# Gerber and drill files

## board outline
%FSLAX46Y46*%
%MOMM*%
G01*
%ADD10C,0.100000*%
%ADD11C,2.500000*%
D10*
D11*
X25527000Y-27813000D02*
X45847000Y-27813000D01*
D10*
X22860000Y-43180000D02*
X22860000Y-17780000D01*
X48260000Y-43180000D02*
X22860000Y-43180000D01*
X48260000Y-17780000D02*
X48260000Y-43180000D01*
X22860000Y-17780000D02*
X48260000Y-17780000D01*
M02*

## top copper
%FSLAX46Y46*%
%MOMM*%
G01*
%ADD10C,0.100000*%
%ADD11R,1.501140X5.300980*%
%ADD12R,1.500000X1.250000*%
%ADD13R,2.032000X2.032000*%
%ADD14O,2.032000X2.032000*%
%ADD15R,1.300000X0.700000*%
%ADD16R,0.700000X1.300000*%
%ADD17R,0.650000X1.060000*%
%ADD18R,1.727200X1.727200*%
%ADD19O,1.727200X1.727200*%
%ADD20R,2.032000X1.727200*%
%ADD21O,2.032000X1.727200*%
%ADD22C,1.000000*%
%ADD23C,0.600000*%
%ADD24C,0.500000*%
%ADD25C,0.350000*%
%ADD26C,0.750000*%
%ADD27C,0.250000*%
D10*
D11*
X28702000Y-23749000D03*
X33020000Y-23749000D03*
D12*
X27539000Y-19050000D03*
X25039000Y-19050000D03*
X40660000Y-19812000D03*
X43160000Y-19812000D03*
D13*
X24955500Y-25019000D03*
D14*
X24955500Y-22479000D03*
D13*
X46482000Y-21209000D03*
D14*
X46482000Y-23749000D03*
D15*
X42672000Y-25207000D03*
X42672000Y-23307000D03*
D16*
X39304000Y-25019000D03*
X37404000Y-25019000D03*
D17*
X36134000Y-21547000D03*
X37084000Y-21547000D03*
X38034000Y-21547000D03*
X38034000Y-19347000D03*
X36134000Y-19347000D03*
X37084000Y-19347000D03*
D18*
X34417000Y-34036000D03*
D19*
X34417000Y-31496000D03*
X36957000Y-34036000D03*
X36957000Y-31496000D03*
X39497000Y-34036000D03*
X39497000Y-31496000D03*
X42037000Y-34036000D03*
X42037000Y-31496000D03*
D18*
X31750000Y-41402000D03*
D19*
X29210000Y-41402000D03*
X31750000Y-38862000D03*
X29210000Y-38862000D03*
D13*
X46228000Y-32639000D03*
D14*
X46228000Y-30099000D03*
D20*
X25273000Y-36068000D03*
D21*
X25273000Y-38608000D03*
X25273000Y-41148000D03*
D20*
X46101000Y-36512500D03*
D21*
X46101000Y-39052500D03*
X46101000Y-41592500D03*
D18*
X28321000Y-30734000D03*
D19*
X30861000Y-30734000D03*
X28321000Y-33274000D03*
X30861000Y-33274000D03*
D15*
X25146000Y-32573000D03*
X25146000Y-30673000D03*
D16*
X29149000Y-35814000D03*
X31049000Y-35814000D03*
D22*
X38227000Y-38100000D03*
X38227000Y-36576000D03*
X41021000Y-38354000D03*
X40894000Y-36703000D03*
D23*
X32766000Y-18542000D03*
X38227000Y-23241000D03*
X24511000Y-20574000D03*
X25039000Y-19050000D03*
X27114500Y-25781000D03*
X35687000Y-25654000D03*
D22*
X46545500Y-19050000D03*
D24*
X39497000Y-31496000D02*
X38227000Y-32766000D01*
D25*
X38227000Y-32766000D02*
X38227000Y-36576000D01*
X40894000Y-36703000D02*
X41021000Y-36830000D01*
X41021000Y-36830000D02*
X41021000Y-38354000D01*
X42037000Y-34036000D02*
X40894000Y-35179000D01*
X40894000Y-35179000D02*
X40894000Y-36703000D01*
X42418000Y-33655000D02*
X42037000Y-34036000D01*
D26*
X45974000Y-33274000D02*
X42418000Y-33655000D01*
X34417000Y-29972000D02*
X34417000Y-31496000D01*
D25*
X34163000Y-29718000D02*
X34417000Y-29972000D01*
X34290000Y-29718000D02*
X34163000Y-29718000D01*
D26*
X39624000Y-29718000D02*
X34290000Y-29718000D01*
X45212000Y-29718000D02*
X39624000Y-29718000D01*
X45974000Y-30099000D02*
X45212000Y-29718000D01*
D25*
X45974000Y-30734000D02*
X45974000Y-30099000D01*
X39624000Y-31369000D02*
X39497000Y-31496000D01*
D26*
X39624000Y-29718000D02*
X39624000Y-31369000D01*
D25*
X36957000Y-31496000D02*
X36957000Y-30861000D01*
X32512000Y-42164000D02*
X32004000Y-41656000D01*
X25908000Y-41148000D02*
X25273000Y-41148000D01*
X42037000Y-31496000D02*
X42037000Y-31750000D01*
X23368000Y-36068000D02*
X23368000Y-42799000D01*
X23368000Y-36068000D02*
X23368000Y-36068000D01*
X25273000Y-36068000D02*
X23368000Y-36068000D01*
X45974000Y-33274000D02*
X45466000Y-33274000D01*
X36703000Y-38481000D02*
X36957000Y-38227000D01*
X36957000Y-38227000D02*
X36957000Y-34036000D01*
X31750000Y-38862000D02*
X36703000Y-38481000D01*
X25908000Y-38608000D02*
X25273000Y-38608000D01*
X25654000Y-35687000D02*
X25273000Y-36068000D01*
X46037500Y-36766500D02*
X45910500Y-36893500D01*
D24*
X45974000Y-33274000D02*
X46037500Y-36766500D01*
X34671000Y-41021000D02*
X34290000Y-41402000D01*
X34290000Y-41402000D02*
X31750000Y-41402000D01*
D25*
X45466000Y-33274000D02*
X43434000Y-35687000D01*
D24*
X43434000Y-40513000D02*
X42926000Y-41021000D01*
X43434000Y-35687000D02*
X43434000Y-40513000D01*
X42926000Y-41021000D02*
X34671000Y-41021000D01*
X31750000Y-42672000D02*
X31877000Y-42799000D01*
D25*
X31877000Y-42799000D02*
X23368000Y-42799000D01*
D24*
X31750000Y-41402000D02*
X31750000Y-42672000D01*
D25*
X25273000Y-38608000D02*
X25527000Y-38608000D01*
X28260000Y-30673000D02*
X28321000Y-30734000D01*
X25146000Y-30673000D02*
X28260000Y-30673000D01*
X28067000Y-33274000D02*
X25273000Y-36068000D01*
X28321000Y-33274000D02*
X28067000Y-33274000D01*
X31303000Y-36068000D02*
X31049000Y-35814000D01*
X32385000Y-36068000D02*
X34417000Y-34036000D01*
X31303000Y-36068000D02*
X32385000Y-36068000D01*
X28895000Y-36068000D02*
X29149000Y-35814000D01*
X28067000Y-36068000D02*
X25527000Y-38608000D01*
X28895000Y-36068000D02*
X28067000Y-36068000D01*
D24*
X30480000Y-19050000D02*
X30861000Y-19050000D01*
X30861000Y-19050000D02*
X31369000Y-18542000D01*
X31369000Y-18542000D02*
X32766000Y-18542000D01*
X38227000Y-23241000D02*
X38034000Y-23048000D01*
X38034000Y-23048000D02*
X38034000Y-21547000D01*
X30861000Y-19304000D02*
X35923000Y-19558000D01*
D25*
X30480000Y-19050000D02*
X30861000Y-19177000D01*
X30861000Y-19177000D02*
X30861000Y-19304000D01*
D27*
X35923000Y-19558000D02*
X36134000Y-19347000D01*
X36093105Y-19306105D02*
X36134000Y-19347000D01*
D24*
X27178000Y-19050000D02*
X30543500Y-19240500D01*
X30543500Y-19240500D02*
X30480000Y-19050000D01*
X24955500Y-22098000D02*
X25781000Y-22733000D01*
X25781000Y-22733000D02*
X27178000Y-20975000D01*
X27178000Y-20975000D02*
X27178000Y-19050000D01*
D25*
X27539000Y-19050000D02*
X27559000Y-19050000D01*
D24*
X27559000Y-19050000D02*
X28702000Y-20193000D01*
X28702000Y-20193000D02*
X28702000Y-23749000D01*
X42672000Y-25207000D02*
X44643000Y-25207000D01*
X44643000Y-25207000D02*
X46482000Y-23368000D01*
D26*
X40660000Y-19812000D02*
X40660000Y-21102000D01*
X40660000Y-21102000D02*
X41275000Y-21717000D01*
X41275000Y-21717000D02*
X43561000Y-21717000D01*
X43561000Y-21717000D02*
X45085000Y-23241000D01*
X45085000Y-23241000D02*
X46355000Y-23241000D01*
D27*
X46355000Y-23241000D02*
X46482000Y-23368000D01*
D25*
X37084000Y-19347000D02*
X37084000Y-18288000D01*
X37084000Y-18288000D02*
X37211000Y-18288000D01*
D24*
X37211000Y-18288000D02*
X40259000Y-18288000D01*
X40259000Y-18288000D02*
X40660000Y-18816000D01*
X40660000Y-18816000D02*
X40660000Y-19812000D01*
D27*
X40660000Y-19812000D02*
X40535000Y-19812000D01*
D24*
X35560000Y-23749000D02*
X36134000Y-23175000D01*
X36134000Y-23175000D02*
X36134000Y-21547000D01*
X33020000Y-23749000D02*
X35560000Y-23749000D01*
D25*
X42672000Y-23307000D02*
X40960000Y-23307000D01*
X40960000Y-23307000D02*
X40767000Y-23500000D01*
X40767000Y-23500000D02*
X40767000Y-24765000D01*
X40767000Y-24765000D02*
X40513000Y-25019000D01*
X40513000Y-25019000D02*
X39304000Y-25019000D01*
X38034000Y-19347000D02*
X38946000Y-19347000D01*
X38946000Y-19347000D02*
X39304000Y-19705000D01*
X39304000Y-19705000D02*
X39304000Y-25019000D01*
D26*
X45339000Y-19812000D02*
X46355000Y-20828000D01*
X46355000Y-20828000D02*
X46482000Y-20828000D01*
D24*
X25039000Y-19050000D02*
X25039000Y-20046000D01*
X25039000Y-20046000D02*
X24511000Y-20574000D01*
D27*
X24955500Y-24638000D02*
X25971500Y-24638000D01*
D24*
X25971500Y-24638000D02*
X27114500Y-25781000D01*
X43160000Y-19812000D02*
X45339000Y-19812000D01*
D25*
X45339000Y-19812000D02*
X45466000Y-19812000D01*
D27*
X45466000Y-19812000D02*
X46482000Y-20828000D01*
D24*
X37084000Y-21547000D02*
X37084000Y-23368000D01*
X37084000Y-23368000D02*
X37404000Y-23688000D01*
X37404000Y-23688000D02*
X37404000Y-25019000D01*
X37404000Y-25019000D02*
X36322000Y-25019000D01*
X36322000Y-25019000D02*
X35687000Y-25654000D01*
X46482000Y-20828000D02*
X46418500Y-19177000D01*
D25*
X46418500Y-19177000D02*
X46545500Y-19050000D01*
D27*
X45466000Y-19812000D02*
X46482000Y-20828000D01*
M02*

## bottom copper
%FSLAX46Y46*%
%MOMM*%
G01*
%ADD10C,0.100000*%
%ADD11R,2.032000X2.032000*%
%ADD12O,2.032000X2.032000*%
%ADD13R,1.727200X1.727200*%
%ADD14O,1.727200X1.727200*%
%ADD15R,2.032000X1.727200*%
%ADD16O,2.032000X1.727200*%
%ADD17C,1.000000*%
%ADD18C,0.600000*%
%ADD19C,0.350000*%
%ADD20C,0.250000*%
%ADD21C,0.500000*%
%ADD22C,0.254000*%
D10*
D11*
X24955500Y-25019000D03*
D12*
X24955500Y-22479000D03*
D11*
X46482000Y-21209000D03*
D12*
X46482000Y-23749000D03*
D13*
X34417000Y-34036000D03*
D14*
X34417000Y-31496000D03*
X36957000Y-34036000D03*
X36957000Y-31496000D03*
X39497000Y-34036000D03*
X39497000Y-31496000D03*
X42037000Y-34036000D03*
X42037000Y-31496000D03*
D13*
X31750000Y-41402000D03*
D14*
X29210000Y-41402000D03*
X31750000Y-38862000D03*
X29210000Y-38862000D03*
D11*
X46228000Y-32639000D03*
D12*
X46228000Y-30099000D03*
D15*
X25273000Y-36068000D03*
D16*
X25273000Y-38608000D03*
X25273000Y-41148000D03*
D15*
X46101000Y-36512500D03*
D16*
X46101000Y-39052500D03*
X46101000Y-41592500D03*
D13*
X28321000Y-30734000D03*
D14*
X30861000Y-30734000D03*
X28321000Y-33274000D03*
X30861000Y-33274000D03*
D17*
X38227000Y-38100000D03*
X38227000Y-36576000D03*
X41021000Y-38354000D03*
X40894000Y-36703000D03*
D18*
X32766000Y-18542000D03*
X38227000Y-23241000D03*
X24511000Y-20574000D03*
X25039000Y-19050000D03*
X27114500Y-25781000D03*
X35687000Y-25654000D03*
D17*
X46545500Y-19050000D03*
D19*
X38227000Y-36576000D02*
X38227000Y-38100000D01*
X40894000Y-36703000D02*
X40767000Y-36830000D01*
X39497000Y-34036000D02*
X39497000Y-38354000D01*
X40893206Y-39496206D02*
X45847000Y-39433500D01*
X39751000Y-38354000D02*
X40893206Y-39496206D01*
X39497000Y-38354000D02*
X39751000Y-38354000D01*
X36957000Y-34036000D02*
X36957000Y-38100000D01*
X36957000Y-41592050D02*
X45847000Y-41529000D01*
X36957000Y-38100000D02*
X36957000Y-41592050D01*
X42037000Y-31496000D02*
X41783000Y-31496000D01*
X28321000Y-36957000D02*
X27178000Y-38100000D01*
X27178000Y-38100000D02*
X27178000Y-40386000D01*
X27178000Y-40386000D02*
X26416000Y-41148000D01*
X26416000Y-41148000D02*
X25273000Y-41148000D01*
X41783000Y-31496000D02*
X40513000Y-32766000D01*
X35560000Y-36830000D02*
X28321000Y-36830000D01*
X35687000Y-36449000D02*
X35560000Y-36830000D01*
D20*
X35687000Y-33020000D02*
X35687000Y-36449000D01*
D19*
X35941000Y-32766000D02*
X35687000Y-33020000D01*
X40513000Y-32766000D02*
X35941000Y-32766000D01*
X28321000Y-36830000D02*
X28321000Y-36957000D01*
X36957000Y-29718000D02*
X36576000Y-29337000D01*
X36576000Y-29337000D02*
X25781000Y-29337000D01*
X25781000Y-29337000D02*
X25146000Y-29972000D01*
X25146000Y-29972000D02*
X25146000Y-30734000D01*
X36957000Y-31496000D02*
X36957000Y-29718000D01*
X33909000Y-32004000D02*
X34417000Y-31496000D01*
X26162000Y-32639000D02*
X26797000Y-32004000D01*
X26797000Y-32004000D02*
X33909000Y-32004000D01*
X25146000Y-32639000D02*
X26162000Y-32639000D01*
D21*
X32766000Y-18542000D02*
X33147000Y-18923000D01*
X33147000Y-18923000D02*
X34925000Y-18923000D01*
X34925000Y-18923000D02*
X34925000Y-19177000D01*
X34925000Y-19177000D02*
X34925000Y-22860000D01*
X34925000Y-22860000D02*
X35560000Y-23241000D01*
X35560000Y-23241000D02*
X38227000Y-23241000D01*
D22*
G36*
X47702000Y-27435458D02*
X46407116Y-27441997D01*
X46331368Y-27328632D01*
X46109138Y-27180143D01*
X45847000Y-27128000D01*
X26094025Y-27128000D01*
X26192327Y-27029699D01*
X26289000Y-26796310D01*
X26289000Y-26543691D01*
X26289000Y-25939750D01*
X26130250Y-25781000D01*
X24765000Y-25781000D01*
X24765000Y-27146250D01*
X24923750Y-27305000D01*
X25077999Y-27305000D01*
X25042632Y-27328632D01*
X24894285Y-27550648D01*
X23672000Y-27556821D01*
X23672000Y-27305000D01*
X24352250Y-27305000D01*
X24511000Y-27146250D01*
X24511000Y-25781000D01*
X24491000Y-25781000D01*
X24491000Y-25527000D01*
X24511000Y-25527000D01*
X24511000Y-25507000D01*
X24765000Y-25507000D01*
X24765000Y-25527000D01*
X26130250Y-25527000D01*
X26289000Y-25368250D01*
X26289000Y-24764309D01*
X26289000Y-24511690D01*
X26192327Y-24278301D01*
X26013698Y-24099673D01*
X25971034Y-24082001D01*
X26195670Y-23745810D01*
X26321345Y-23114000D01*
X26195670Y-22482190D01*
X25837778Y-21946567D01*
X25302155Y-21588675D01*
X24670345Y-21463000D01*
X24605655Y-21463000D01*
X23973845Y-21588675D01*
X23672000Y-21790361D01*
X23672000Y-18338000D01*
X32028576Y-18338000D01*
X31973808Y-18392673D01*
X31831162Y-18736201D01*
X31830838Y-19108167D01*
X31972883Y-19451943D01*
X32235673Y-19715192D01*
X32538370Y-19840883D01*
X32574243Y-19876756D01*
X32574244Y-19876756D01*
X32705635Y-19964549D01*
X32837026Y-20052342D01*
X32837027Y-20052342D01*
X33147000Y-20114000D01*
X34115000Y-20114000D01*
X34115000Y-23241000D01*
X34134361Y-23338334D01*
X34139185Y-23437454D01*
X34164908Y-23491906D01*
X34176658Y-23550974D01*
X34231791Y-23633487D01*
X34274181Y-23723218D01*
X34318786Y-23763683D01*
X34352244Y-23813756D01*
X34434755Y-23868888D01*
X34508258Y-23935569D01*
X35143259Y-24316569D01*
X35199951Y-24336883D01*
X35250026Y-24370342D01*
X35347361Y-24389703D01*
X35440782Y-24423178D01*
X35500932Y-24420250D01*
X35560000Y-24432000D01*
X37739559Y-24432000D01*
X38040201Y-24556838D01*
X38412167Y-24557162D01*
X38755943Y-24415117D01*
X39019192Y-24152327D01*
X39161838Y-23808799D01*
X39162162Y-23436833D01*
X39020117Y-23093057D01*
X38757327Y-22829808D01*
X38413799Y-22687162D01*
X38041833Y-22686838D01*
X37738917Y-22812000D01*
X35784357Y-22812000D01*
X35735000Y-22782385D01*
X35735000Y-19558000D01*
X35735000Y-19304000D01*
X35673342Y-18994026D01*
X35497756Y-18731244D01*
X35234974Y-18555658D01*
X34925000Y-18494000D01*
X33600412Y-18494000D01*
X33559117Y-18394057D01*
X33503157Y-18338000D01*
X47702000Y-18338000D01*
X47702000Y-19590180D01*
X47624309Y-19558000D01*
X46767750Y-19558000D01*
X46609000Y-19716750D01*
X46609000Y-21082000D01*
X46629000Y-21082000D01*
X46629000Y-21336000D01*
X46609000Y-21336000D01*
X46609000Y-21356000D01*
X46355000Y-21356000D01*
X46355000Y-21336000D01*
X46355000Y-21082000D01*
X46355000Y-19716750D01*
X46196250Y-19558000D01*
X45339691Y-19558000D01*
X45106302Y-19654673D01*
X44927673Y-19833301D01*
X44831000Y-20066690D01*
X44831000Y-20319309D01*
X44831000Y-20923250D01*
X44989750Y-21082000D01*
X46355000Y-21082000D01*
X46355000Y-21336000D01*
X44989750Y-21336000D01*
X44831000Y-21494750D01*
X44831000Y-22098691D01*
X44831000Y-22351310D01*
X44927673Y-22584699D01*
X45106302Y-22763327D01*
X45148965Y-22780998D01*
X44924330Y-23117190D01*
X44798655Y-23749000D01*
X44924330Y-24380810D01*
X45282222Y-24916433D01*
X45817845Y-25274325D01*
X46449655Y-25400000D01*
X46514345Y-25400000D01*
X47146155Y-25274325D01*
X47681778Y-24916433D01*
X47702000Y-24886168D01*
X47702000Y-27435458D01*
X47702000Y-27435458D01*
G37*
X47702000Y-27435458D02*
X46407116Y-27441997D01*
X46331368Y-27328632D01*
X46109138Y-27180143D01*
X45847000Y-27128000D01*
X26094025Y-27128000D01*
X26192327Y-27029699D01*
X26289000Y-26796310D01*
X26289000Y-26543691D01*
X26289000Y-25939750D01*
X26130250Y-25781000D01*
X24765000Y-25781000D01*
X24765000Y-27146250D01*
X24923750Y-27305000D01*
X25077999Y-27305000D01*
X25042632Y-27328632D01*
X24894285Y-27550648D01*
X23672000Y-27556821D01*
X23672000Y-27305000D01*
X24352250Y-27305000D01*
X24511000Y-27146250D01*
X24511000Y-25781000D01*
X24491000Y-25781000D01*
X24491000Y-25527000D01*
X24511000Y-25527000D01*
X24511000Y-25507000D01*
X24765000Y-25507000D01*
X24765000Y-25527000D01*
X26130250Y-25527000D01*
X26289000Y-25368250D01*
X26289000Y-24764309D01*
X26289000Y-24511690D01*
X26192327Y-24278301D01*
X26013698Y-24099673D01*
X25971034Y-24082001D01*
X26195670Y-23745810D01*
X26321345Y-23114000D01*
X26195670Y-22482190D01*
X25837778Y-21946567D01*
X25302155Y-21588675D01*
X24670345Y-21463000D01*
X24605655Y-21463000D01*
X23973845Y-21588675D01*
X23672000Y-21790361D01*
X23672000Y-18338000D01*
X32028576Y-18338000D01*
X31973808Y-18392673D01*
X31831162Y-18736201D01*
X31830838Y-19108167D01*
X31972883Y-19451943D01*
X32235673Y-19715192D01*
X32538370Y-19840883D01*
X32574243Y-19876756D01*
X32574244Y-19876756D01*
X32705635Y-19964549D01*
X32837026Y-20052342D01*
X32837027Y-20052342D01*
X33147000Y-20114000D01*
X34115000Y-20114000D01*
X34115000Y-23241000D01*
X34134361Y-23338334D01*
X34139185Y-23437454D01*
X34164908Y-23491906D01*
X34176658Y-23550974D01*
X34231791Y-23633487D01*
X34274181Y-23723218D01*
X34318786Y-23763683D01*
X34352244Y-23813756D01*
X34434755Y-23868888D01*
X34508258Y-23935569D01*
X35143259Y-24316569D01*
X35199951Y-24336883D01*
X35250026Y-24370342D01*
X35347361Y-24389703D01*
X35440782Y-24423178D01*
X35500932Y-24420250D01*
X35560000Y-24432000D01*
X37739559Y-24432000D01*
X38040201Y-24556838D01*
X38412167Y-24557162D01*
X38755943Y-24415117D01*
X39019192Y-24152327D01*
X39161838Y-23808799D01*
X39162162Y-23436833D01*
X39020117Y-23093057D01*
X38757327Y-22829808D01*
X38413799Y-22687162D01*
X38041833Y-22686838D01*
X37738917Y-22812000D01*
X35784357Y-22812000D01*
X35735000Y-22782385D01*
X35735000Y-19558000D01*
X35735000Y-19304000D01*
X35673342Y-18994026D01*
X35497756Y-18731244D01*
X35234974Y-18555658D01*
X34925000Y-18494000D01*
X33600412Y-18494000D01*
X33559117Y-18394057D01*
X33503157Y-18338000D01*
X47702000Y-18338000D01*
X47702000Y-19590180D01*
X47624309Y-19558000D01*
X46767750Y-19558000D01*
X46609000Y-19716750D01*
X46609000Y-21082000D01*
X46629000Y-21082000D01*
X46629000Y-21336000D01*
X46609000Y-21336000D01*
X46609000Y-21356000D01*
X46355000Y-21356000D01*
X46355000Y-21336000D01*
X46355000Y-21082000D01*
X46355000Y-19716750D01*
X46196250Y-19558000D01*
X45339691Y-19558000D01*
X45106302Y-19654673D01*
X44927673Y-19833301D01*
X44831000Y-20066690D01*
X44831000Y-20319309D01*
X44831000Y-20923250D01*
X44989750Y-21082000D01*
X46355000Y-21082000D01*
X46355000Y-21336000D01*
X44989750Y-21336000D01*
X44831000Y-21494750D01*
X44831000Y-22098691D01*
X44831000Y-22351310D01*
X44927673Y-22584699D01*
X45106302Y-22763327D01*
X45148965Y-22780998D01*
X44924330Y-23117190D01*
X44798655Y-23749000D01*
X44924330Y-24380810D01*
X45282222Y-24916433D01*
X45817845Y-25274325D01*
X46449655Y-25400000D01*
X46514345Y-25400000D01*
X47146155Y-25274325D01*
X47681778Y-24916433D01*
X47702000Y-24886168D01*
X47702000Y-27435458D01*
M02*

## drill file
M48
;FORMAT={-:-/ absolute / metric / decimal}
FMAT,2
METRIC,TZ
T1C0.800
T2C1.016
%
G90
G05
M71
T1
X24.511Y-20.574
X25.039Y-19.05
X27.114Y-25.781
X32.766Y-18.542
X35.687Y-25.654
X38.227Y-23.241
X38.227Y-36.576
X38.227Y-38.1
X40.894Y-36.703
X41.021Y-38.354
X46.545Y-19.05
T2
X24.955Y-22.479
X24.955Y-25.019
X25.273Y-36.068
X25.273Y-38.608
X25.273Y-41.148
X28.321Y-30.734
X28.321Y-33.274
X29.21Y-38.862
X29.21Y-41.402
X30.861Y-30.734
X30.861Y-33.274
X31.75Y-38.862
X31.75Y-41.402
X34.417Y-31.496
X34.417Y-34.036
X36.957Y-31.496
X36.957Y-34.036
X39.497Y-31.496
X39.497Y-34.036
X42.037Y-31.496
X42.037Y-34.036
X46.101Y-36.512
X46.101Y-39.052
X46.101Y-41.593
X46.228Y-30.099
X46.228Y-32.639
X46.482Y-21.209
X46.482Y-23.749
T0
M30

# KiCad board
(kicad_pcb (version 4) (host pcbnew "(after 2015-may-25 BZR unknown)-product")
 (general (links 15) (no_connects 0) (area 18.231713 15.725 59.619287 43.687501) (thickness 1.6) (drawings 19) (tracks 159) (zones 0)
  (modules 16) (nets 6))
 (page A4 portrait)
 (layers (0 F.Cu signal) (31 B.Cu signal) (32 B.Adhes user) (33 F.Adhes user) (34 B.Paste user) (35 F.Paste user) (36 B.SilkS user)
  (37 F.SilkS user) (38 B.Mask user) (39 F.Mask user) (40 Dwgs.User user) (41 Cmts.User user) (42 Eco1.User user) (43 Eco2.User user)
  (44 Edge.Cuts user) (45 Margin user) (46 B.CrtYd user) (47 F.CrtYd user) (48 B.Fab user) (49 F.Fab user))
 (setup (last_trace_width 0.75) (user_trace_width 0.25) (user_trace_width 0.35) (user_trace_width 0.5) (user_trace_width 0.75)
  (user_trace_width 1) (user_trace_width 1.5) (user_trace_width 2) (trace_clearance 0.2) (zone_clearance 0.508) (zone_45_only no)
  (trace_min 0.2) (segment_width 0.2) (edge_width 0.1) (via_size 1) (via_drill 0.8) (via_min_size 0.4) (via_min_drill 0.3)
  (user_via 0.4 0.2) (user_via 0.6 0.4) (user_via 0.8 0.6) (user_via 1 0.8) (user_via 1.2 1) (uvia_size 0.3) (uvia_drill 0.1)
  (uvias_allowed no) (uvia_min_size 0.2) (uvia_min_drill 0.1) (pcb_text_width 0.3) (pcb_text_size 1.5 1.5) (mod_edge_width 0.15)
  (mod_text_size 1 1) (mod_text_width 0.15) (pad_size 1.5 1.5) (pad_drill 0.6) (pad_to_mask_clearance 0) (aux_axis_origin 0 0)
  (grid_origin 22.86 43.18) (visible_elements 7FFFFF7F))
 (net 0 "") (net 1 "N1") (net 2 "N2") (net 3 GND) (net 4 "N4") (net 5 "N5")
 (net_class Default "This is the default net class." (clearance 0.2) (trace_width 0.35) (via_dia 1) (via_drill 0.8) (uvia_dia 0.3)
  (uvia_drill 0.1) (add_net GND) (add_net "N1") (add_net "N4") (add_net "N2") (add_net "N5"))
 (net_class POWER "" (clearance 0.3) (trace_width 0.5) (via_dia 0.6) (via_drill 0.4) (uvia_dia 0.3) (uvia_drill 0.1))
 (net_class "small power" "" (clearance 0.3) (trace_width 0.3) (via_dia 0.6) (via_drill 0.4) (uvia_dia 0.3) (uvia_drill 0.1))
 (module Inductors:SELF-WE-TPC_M (layer F.Cu) (at 30.861 23.749)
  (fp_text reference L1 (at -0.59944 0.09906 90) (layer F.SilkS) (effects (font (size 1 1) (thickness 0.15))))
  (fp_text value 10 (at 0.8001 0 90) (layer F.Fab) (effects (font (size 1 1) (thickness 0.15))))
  (pad 1 smd rect (at -2.159 0) (size 1.50114 5.30098) (layers F.Cu F.Paste F.Mask) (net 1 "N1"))
  (pad 2 smd rect (at 2.159 0) (size 1.50114 5.30098) (layers F.Cu F.Paste F.Mask) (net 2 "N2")))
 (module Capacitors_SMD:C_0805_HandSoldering (layer F.Cu) (at 26.289 19.05 180)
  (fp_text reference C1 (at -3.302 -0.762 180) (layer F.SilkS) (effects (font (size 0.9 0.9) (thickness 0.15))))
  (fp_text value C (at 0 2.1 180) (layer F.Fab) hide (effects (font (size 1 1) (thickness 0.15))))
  (pad 1 smd rect (at -1.25 0 180) (size 1.5 1.25) (layers F.Cu F.Paste F.Mask) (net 1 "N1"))
  (pad 2 smd rect (at 1.25 0 180) (size 1.5 1.25) (layers F.Cu F.Paste F.Mask) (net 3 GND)))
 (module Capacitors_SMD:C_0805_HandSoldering (layer F.Cu) (at 41.91 19.812)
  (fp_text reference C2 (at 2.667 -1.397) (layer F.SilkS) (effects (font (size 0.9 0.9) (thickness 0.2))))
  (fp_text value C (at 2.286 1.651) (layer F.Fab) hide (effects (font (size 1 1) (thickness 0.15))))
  (pad 1 smd rect (at -1.25 0) (size 1.5 1.25) (layers F.Cu F.Paste F.Mask) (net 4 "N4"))
  (pad 2 smd rect (at 1.25 0) (size 1.5 1.25) (layers F.Cu F.Paste F.Mask) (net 3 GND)))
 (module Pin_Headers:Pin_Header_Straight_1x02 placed (layer F.Cu) (at 24.9555 25.019 180)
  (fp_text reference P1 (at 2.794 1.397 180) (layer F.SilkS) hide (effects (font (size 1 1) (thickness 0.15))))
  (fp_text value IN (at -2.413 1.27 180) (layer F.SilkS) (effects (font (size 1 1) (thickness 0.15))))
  (pad 1 thru_hole rect (at 0 0 180) (size 2.032 2.032) (drill 1.016) (layers *.Cu *.Mask F.SilkS) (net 3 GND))
  (pad 2 thru_hole oval (at 0 2.54 180) (size 2.032 2.032) (drill 1.016) (layers *.Cu *.Mask F.SilkS) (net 1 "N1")))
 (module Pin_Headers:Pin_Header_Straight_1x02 (layer F.Cu) (at 46.482 21.209)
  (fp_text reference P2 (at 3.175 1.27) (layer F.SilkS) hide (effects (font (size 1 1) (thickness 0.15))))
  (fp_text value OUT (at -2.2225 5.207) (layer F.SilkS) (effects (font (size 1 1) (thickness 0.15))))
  (pad 1 thru_hole rect (at 0 0) (size 2.032 2.032) (drill 1.016) (layers *.Cu *.Mask F.SilkS) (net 3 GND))
  (pad 2 thru_hole oval (at 0 2.54) (size 2.032 2.032) (drill 1.016) (layers *.Cu *.Mask F.SilkS) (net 4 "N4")))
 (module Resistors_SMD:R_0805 (layer F.Cu) (at 42.672 24.257 90)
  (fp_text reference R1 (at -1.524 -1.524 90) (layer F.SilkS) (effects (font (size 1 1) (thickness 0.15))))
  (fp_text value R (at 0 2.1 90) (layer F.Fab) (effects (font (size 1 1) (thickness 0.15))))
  (pad 1 smd rect (at -0.95 0 90) (size 0.7 1.3) (layers F.Cu F.Paste F.Mask) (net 4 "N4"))
  (pad 2 smd rect (at 0.95 0 90) (size 0.7 1.3) (layers F.Cu F.Paste F.Mask) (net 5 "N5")))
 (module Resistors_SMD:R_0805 (layer F.Cu) (at 38.354 25.019 180)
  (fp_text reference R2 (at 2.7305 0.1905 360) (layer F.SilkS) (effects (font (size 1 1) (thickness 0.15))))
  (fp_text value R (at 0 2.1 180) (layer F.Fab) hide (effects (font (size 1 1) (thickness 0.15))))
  (pad 1 smd rect (at -0.95 0 180) (size 0.7 1.3) (layers F.Cu F.Paste F.Mask) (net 5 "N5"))
  (pad 2 smd rect (at 0.95 0 180) (size 0.7 1.3) (layers F.Cu F.Paste F.Mask) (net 3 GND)))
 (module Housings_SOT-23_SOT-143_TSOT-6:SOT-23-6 (layer F.Cu) (at 37.084 20.447 90)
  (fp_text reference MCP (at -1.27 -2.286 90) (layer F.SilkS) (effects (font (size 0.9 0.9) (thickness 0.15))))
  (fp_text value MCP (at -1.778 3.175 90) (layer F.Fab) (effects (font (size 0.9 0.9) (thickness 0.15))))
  (pad 1 smd rect (at -1.1 -0.95 90) (size 1.06 0.65) (layers F.Cu F.Paste F.Mask) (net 2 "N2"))
  (pad 2 smd rect (at -1.1 0 90) (size 1.06 0.65) (layers F.Cu F.Paste F.Mask) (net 3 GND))
  (pad 3 smd rect (at -1.1 0.95 90) (size 1.06 0.65) (layers F.Cu F.Paste F.Mask) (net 1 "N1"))
  (pad 4 smd rect (at 1.1 0.95 90) (size 1.06 0.65) (layers F.Cu F.Paste F.Mask) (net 5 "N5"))
  (pad 6 smd rect (at 1.1 -0.95 90) (size 1.06 0.65) (layers F.Cu F.Paste F.Mask) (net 1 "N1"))
  (pad 5 smd rect (at 1.1 0 90) (size 1.06 0.65) (layers F.Cu F.Paste F.Mask) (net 4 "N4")))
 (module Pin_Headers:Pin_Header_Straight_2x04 (layer F.Cu) (at 34.417 34.036 90)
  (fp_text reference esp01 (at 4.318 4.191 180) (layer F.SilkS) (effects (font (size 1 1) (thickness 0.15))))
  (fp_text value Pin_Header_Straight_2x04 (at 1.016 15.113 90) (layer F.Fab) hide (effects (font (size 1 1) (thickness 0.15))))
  (pad 1 thru_hole rect (at 0 0 90) (size 1.7272 1.7272) (drill 1.016) (layers *.Cu *.Mask F.SilkS))
  (pad 2 thru_hole oval (at 2.54 0 90) (size 1.7272 1.7272) (drill 1.016) (layers *.Cu *.Mask F.SilkS))
  (pad 3 thru_hole oval (at 0 2.54 90) (size 1.7272 1.7272) (drill 1.016) (layers *.Cu *.Mask F.SilkS))
  (pad 4 thru_hole oval (at 2.54 2.54 90) (size 1.7272 1.7272) (drill 1.016) (layers *.Cu *.Mask F.SilkS))
  (pad 5 thru_hole oval (at 0 5.08 90) (size 1.7272 1.7272) (drill 1.016) (layers *.Cu *.Mask F.SilkS))
  (pad 6 thru_hole oval (at 2.54 5.08 90) (size 1.7272 1.7272) (drill 1.016) (layers *.Cu *.Mask F.SilkS))
  (pad 7 thru_hole oval (at 0 7.62 90) (size 1.7272 1.7272) (drill 1.016) (layers *.Cu *.Mask F.SilkS))
  (pad 8 thru_hole oval (at 2.54 7.62 90) (size 1.7272 1.7272) (drill 1.016) (layers *.Cu *.Mask F.SilkS)))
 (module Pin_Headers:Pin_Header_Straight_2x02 (layer F.Cu) (at 31.75 41.402 180)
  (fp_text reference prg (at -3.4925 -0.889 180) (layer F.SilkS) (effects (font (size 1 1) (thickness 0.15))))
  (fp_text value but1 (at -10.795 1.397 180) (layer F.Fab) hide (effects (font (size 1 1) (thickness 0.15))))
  (pad 1 thru_hole rect (at 0 0 180) (size 1.7272 1.7272) (drill 1.016) (layers *.Cu *.Mask F.SilkS))
  (pad 2 thru_hole oval (at 2.54 0 180) (size 1.7272 1.7272) (drill 1.016) (layers *.Cu *.Mask F.SilkS))
  (pad 3 thru_hole oval (at 0 2.54 180) (size 1.7272 1.7272) (drill 1.016) (layers *.Cu *.Mask F.SilkS))
  (pad 4 thru_hole oval (at 2.54 2.54 180) (size 1.7272 1.7272) (drill 1.016) (layers *.Cu *.Mask F.SilkS)))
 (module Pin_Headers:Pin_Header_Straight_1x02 (layer F.Cu) (at 46.228 32.639 180)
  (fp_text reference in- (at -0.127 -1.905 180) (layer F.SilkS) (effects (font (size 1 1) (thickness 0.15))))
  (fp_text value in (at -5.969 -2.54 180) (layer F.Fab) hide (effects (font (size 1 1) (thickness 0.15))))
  (pad 1 thru_hole rect (at 0 0 180) (size 2.032 2.032) (drill 1.016) (layers *.Cu *.Mask F.SilkS))
  (pad 2 thru_hole oval (at 0 2.54 180) (size 2.032 2.032) (drill 1.016) (layers *.Cu *.Mask F.SilkS)))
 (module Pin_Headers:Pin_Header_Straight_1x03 (layer F.Cu) (at 25.273 36.068)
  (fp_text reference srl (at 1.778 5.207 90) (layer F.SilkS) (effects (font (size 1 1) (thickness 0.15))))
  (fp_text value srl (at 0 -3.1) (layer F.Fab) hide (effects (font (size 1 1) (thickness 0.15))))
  (pad 1 thru_hole rect (at 0 0) (size 2.032 1.7272) (drill 1.016) (layers *.Cu *.Mask F.SilkS))
  (pad 2 thru_hole oval (at 0 2.54) (size 2.032 1.7272) (drill 1.016) (layers *.Cu *.Mask F.SilkS))
  (pad 3 thru_hole oval (at 0 5.08) (size 2.032 1.7272) (drill 1.016) (layers *.Cu *.Mask F.SilkS)))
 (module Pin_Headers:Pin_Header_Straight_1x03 (layer F.Cu) (at 46.101 36.5125)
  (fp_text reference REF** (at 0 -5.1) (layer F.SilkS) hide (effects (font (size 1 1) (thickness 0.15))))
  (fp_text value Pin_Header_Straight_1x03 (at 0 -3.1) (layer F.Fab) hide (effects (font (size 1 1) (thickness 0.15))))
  (pad 1 thru_hole rect (at 0 0) (size 2.032 1.7272) (drill 1.016) (layers *.Cu *.Mask F.SilkS))
  (pad 2 thru_hole oval (at 0 2.54) (size 2.032 1.7272) (drill 1.016) (layers *.Cu *.Mask F.SilkS))
  (pad 3 thru_hole oval (at 0 5.08) (size 2.032 1.7272) (drill 1.016) (layers *.Cu *.Mask F.SilkS)))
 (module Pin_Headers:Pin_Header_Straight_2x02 (layer F.Cu) (at 28.321 30.734)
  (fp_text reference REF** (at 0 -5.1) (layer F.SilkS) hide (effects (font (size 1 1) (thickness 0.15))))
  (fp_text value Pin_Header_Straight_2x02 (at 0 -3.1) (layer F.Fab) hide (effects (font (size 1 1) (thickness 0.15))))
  (pad 1 thru_hole rect (at 0 0) (size 1.7272 1.7272) (drill 1.016) (layers *.Cu *.Mask F.SilkS))
  (pad 2 thru_hole oval (at 2.54 0) (size 1.7272 1.7272) (drill 1.016) (layers *.Cu *.Mask F.SilkS))
  (pad 3 thru_hole oval (at 0 2.54) (size 1.7272 1.7272) (drill 1.016) (layers *.Cu *.Mask F.SilkS))
  (pad 4 thru_hole oval (at 2.54 2.54) (size 1.7272 1.7272) (drill 1.016) (layers *.Cu *.Mask F.SilkS)))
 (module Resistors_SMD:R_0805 (layer F.Cu) (at 25.146 31.623 90)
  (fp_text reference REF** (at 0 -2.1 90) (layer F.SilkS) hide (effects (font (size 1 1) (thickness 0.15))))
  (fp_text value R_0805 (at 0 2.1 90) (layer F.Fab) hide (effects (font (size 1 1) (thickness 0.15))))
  (pad 1 smd rect (at -0.95 0 90) (size 0.7 1.3) (layers F.Cu F.Paste F.Mask))
  (pad 2 smd rect (at 0.95 0 90) (size 0.7 1.3) (layers F.Cu F.Paste F.Mask)))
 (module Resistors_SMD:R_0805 (layer F.Cu) (at 30.099 35.814)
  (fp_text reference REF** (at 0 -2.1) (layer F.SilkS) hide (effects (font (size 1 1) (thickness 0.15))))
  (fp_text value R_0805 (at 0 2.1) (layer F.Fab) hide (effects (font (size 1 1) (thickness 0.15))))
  (pad 1 smd rect (at -0.95 0) (size 0.7 1.3) (layers F.Cu F.Paste F.Mask))
  (pad 2 smd rect (at 0.95 0) (size 0.7 1.3) (layers F.Cu F.Paste F.Mask)))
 (gr_line (start 25.527 27.813) (end 45.847 27.813) (angle 90) (layer Edge.Cuts) (width 2.5))
 (gr_line (start 22.86 43.18) (end 22.86 17.78) (angle 90) (layer Edge.Cuts) (width 0.1))
 (gr_line (start 48.26 43.18) (end 22.86 43.18) (angle 90) (layer Edge.Cuts) (width 0.1))
 (gr_line (start 48.26 17.78) (end 48.26 43.18) (angle 90) (layer Edge.Cuts) (width 0.1))
 (gr_line (start 22.86 17.78) (end 48.26 17.78) (angle 90) (layer Edge.Cuts) (width 0.1))
 (segment (start 39.497 31.496) (end 38.227 32.766) (width 0.5) (layer F.Cu) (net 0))
 (via (at 38.227 38.1) (size 1) (layers F.Cu B.Cu) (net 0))
 (segment (start 38.227 36.576) (end 38.227 38.1) (width 0.35) (layer B.Cu) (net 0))
 (via (at 38.227 36.576) (size 1) (layers F.Cu B.Cu) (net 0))
 (segment (start 38.227 32.766) (end 38.227 36.576) (width 0.35) (layer F.Cu) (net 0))
 (segment (start 40.894 36.703) (end 41.021 36.83) (width 0.35) (layer F.Cu) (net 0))
 (via (at 41.021 38.354) (size 1) (layers F.Cu B.Cu) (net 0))
 (segment (start 41.021 36.83) (end 41.021 38.354) (width 0.35) (layer F.Cu) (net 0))
 (segment (start 42.037 34.036) (end 40.894 35.179) (width 0.35) (layer F.Cu) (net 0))
 (segment (start 40.894 36.703) (end 40.767 36.83) (width 0.35) (layer B.Cu) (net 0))
 (via (at 40.894 36.703) (size 1) (layers F.Cu B.Cu) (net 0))
 (segment (start 40.894 35.179) (end 40.894 36.703) (width 0.35) (layer F.Cu) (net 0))
 (segment (start 42.418 33.655) (end 42.037 34.036) (width 0.35) (layer F.Cu) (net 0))
 (segment (start 45.974 33.274) (end 42.418 33.655) (width 0.75) (layer F.Cu) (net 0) (status 10))
 (segment (start 34.417 29.972) (end 34.417 31.496) (width 0.75) (layer F.Cu) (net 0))
 (segment (start 34.163 29.718) (end 34.417 29.972) (width 0.35) (layer F.Cu) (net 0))
 (segment (start 34.29 29.718) (end 34.163 29.718) (width 0.35) (layer F.Cu) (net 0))
 (segment (start 39.624 29.718) (end 34.29 29.718) (width 0.75) (layer F.Cu) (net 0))
 (segment (start 45.212 29.718) (end 39.624 29.718) (width 0.75) (layer F.Cu) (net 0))
 (segment (start 45.974 30.099) (end 45.212 29.718) (width 0.75) (layer F.Cu) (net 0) (status 10))
 (segment (start 45.974 30.734) (end 45.974 30.099) (width 0.35) (layer F.Cu) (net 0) (status 30))
 (segment (start 39.624 31.369) (end 39.497 31.496) (width 0.35) (layer F.Cu) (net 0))
 (segment (start 39.624 29.718) (end 39.624 31.369) (width 0.75) (layer F.Cu) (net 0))
 (segment (start 36.957 31.496) (end 36.957 30.861) (width 0.35) (layer F.Cu) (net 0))
 (segment (start 32.512 42.164) (end 32.004 41.656) (width 0.35) (layer F.Cu) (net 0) (status 30))
 (segment (start 25.908 41.148) (end 25.273 41.148) (width 0.35) (layer F.Cu) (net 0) (status 30))
 (segment (start 42.037 31.496) (end 42.037 31.75) (width 0.35) (layer F.Cu) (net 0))
 (segment (start 23.368 36.068) (end 23.368 42.799) (width 0.35) (layer F.Cu) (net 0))
 (segment (start 23.368 36.068) (end 23.368 36.068) (width 0.35) (layer F.Cu) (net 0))
 (segment (start 25.273 36.068) (end 23.368 36.068) (width 0.35) (layer F.Cu) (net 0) (status 10))
 (segment (start 45.974 33.274) (end 45.466 33.274) (width 0.35) (layer F.Cu) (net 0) (status 30))
 (segment (start 36.703 38.481) (end 36.957 38.227) (width 0.35) (layer F.Cu) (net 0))
 (segment (start 36.957 38.227) (end 36.957 34.036) (width 0.35) (layer F.Cu) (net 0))
 (segment (start 31.75 38.862) (end 36.703 38.481) (width 0.35) (layer F.Cu) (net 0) (status 10))
 (segment (start 25.908 38.608) (end 25.273 38.608) (width 0.35) (layer F.Cu) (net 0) (status 30))
 (segment (start 25.654 35.687) (end 25.273 36.068) (width 0.35) (layer F.Cu) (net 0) (status 30))
 (segment (start 46.0375 36.7665) (end 45.9105 36.8935) (width 0.35) (layer F.Cu) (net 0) (status 30))
 (segment (start 45.974 33.274) (end 46.0375 36.7665) (width 0.5) (layer F.Cu) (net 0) (status 20))
 (segment (start 39.497 34.036) (end 39.497 38.354) (width 0.35) (layer B.Cu) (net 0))
 (segment (start 40.893206 39.496206) (end 45.847 39.4335) (width 0.35) (layer B.Cu) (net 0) (status 20))
 (segment (start 39.751 38.354) (end 40.893206 39.496206) (width 0.35) (layer B.Cu) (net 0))
 (segment (start 39.497 38.354) (end 39.751 38.354) (width 0.35) (layer B.Cu) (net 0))
 (segment (start 36.957 34.036) (end 36.957 38.1) (width 0.35) (layer B.Cu) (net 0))
 (segment (start 36.957 41.59205) (end 45.847 41.529) (width 0.35) (layer B.Cu) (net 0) (status 20))
 (segment (start 36.957 38.1) (end 36.957 41.59205) (width 0.35) (layer B.Cu) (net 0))
 (segment (start 42.037 31.496) (end 41.783 31.496) (width 0.35) (layer B.Cu) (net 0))
 (segment (start 34.671 41.021) (end 34.29 41.402) (width 0.5) (layer F.Cu) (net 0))
 (segment (start 34.29 41.402) (end 31.75 41.402) (width 0.5) (layer F.Cu) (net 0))
 (segment (start 45.466 33.274) (end 43.434 35.687) (width 0.35) (layer F.Cu) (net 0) (status 10))
 (segment (start 43.434 40.513) (end 42.926 41.021) (width 0.5) (layer F.Cu) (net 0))
 (segment (start 43.434 35.687) (end 43.434 40.513) (width 0.5) (layer F.Cu) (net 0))
 (segment (start 42.926 41.021) (end 34.671 41.021) (width 0.5) (layer F.Cu) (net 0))
 (segment (start 31.75 42.672) (end 31.877 42.799) (width 0.5) (layer F.Cu) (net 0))
 (segment (start 31.877 42.799) (end 23.368 42.799) (width 0.35) (layer F.Cu) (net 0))
 (segment (start 31.75 41.402) (end 31.75 42.672) (width 0.5) (layer F.Cu) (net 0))
 (segment (start 28.321 36.957) (end 27.178 38.1) (width 0.35) (layer B.Cu) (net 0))
 (segment (start 27.178 38.1) (end 27.178 40.386) (width 0.35) (layer B.Cu) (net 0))
 (segment (start 27.178 40.386) (end 26.416 41.148) (width 0.35) (layer B.Cu) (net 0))
 (segment (start 26.416 41.148) (end 25.273 41.148) (width 0.35) (layer B.Cu) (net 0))
 (segment (start 41.783 31.496) (end 40.513 32.766) (width 0.35) (layer B.Cu) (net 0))
 (segment (start 35.56 36.83) (end 28.321 36.83) (width 0.35) (layer B.Cu) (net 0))
 (segment (start 35.687 36.449) (end 35.56 36.83) (width 0.35) (layer B.Cu) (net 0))
 (segment (start 35.687 33.02) (end 35.687 36.449) (width 0.25) (layer B.Cu) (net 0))
 (segment (start 35.941 32.766) (end 35.687 33.02) (width 0.35) (layer B.Cu) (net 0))
 (segment (start 40.513 32.766) (end 35.941 32.766) (width 0.35) (layer B.Cu) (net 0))
 (segment (start 28.321 36.83) (end 28.321 36.957) (width 0.35) (layer B.Cu) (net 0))
 (segment (start 25.273 38.608) (end 25.527 38.608) (width 0.35) (layer F.Cu) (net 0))
 (segment (start 36.957 29.718) (end 36.576 29.337) (width 0.35) (layer B.Cu) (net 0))
 (segment (start 36.576 29.337) (end 25.781 29.337) (width 0.35) (layer B.Cu) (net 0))
 (segment (start 25.781 29.337) (end 25.146 29.972) (width 0.35) (layer B.Cu) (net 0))
 (segment (start 25.146 29.972) (end 25.146 30.734) (width 0.35) (layer B.Cu) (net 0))
 (segment (start 36.957 31.496) (end 36.957 29.718) (width 0.35) (layer B.Cu) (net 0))
 (segment (start 33.909 32.004) (end 34.417 31.496) (width 0.35) (layer B.Cu) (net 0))
 (segment (start 26.162 32.639) (end 26.797 32.004) (width 0.35) (layer B.Cu) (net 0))
 (segment (start 26.797 32.004) (end 33.909 32.004) (width 0.35) (layer B.Cu) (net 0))
 (segment (start 25.146 32.639) (end 26.162 32.639) (width 0.35) (layer B.Cu) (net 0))
 (segment (start 28.26 30.673) (end 28.321 30.734) (width 0.35) (layer F.Cu) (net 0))
 (segment (start 25.146 30.673) (end 28.26 30.673) (width 0.35) (layer F.Cu) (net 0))
 (segment (start 28.067 33.274) (end 25.273 36.068) (width 0.35) (layer F.Cu) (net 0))
 (segment (start 28.321 33.274) (end 28.067 33.274) (width 0.35) (layer F.Cu) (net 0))
 (segment (start 31.303 36.068) (end 31.049 35.814) (width 0.35) (layer F.Cu) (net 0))
 (segment (start 32.385 36.068) (end 34.417 34.036) (width 0.35) (layer F.Cu) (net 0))
 (segment (start 31.303 36.068) (end 32.385 36.068) (width 0.35) (layer F.Cu) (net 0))
 (segment (start 28.895 36.068) (end 29.149 35.814) (width 0.35) (layer F.Cu) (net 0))
 (segment (start 28.067 36.068) (end 25.527 38.608) (width 0.35) (layer F.Cu) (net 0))
 (segment (start 28.895 36.068) (end 28.067 36.068) (width 0.35) (layer F.Cu) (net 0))
 (segment (start 30.48 19.05) (end 30.861 19.05) (width 0.5) (layer F.Cu) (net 1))
 (segment (start 30.861 19.05) (end 31.369 18.542) (width 0.5) (layer F.Cu) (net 1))
 (segment (start 31.369 18.542) (end 32.766 18.542) (width 0.5) (layer F.Cu) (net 1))
 (via (at 32.766 18.542) (size 0.6) (layers F.Cu B.Cu) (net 1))
 (segment (start 32.766 18.542) (end 33.147 18.923) (width 0.5) (layer B.Cu) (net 1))
 (segment (start 33.147 18.923) (end 34.925 18.923) (width 0.5) (layer B.Cu) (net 1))
 (segment (start 34.925 18.923) (end 34.925 19.177) (width 0.5) (layer B.Cu) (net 1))
 (segment (start 34.925 19.177) (end 34.925 22.86) (width 0.5) (layer B.Cu) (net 1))
 (segment (start 34.925 22.86) (end 35.56 23.241) (width 0.5) (layer B.Cu) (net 1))
 (segment (start 35.56 23.241) (end 38.227 23.241) (width 0.5) (layer B.Cu) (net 1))
 (via (at 38.227 23.241) (size 0.6) (layers F.Cu B.Cu) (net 1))
 (segment (start 38.227 23.241) (end 38.034 23.048) (width 0.5) (layer F.Cu) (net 1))
 (segment (start 38.034 23.048) (end 38.034 21.547) (width 0.5) (layer F.Cu) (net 1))
 (segment (start 30.861 19.304) (end 35.923 19.558) (width 0.5) (layer F.Cu) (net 1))
 (segment (start 30.48 19.05) (end 30.861 19.177) (width 0.35) (layer F.Cu) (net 1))
 (segment (start 30.861 19.177) (end 30.861 19.304) (width 0.35) (layer F.Cu) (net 1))
 (segment (start 35.923 19.558) (end 36.134 19.347) (width 0.25) (layer F.Cu) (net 1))
 (segment (start 36.093105 19.306105) (end 36.134 19.347) (width 0.25) (layer F.Cu) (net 1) (status 30))
 (segment (start 27.178 19.05) (end 30.5435 19.2405) (width 0.5) (layer F.Cu) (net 1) (status 10))
 (segment (start 30.5435 19.2405) (end 30.48 19.05) (width 0.5) (layer F.Cu) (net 1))
 (segment (start 24.9555 22.098) (end 25.781 22.733) (width 0.5) (layer F.Cu) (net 1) (status 10))
 (segment (start 25.781 22.733) (end 27.178 20.975) (width 0.5) (layer F.Cu) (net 1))
 (segment (start 27.178 20.975) (end 27.178 19.05) (width 0.5) (layer F.Cu) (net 1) (status 20))
 (segment (start 27.539 19.05) (end 27.559 19.05) (width 0.35) (layer F.Cu) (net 1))
 (segment (start 27.559 19.05) (end 28.702 20.193) (width 0.5) (layer F.Cu) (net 1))
 (segment (start 28.702 20.193) (end 28.702 23.749) (width 0.5) (layer F.Cu) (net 1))
 (segment (start 42.672 25.207) (end 44.643 25.207) (width 0.5) (layer F.Cu) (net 4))
 (segment (start 44.643 25.207) (end 46.482 23.368) (width 0.5) (layer F.Cu) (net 4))
 (segment (start 40.66 19.812) (end 40.66 21.102) (width 0.75) (layer F.Cu) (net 4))
 (segment (start 40.66 21.102) (end 41.275 21.717) (width 0.75) (layer F.Cu) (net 4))
 (segment (start 41.275 21.717) (end 43.561 21.717) (width 0.75) (layer F.Cu) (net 4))
 (segment (start 43.561 21.717) (end 45.085 23.241) (width 0.75) (layer F.Cu) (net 4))
 (segment (start 45.085 23.241) (end 46.355 23.241) (width 0.75) (layer F.Cu) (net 4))
 (segment (start 46.355 23.241) (end 46.482 23.368) (width 0.25) (layer F.Cu) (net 4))
 (segment (start 37.084 19.347) (end 37.084 18.288) (width 0.35) (layer F.Cu) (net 4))
 (segment (start 37.084 18.288) (end 37.211 18.288) (width 0.35) (layer F.Cu) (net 4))
 (segment (start 37.211 18.288) (end 40.259 18.288) (width 0.5) (layer F.Cu) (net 4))
 (segment (start 40.259 18.288) (end 40.66 18.816) (width 0.5) (layer F.Cu) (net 4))
 (segment (start 40.66 18.816) (end 40.66 19.812) (width 0.5) (layer F.Cu) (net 4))
 (segment (start 40.66 19.812) (end 40.535 19.812) (width 0.25) (layer F.Cu) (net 4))
 (segment (start 35.56 23.749) (end 36.134 23.175) (width 0.5) (layer F.Cu) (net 2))
 (segment (start 36.134 23.175) (end 36.134 21.547) (width 0.5) (layer F.Cu) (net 2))
 (segment (start 33.02 23.749) (end 35.56 23.749) (width 0.5) (layer F.Cu) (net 2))
 (segment (start 42.672 23.307) (end 40.96 23.307) (width 0.35) (layer F.Cu) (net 5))
 (segment (start 40.96 23.307) (end 40.767 23.5) (width 0.35) (layer F.Cu) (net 5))
 (segment (start 40.767 23.5) (end 40.767 24.765) (width 0.35) (layer F.Cu) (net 5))
 (segment (start 40.767 24.765) (end 40.513 25.019) (width 0.35) (layer F.Cu) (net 5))
 (segment (start 40.513 25.019) (end 39.304 25.019) (width 0.35) (layer F.Cu) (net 5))
 (segment (start 38.034 19.347) (end 38.946 19.347) (width 0.35) (layer F.Cu) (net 5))
 (segment (start 38.946 19.347) (end 39.304 19.705) (width 0.35) (layer F.Cu) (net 5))
 (segment (start 39.304 19.705) (end 39.304 25.019) (width 0.35) (layer F.Cu) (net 5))
 (segment (start 45.339 19.812) (end 46.355 20.828) (width 0.75) (layer F.Cu) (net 3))
 (segment (start 46.355 20.828) (end 46.482 20.828) (width 0.75) (layer F.Cu) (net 3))
 (segment (start 25.039 19.05) (end 25.039 20.046) (width 0.5) (layer F.Cu) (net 3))
 (segment (start 25.039 20.046) (end 24.511 20.574) (width 0.5) (layer F.Cu) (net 3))
 (via (at 24.511 20.574) (size 0.6) (layers F.Cu B.Cu) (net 3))
 (via (at 25.039 19.05) (size 0.6) (layers F.Cu B.Cu) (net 3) (status 30))
 (segment (start 24.9555 24.638) (end 25.9715 24.638) (width 0.25) (layer F.Cu) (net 3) (status 30))
 (segment (start 25.9715 24.638) (end 27.1145 25.781) (width 0.5) (layer F.Cu) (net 3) (status 10))
 (via (at 27.1145 25.781) (size 0.6) (layers F.Cu B.Cu) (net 3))
 (segment (start 43.16 19.812) (end 45.339 19.812) (width 0.5) (layer F.Cu) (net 3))
 (segment (start 45.339 19.812) (end 45.466 19.812) (width 0.35) (layer F.Cu) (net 3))
 (segment (start 45.466 19.812) (end 46.482 20.828) (width 0.25) (layer F.Cu) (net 3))
 (segment (start 37.084 21.547) (end 37.084 23.368) (width 0.5) (layer F.Cu) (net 3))
 (segment (start 37.084 23.368) (end 37.404 23.688) (width 0.5) (layer F.Cu) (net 3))
 (segment (start 37.404 23.688) (end 37.404 25.019) (width 0.5) (layer F.Cu) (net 3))
 (segment (start 37.404 25.019) (end 36.322 25.019) (width 0.5) (layer F.Cu) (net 3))
 (segment (start 36.322 25.019) (end 35.687 25.654) (width 0.5) (layer F.Cu) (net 3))
 (via (at 35.687 25.654) (size 0.6) (layers F.Cu B.Cu) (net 3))
 (segment (start 46.482 20.828) (end 46.4185 19.177) (width 0.5) (layer F.Cu) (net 3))
 (segment (start 46.4185 19.177) (end 46.5455 19.05) (width 0.35) (layer F.Cu) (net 3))
 (via (at 46.5455 19.05) (size 1) (layers F.Cu B.Cu) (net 3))
 (segment (start 45.466 19.812) (end 46.482 20.828) (width 0.25) (layer F.Cu) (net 3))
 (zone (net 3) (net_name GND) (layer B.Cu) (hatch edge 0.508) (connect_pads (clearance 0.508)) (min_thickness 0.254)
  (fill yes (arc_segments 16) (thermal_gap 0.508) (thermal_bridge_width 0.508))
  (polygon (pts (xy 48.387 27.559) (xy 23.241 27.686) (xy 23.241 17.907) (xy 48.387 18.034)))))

